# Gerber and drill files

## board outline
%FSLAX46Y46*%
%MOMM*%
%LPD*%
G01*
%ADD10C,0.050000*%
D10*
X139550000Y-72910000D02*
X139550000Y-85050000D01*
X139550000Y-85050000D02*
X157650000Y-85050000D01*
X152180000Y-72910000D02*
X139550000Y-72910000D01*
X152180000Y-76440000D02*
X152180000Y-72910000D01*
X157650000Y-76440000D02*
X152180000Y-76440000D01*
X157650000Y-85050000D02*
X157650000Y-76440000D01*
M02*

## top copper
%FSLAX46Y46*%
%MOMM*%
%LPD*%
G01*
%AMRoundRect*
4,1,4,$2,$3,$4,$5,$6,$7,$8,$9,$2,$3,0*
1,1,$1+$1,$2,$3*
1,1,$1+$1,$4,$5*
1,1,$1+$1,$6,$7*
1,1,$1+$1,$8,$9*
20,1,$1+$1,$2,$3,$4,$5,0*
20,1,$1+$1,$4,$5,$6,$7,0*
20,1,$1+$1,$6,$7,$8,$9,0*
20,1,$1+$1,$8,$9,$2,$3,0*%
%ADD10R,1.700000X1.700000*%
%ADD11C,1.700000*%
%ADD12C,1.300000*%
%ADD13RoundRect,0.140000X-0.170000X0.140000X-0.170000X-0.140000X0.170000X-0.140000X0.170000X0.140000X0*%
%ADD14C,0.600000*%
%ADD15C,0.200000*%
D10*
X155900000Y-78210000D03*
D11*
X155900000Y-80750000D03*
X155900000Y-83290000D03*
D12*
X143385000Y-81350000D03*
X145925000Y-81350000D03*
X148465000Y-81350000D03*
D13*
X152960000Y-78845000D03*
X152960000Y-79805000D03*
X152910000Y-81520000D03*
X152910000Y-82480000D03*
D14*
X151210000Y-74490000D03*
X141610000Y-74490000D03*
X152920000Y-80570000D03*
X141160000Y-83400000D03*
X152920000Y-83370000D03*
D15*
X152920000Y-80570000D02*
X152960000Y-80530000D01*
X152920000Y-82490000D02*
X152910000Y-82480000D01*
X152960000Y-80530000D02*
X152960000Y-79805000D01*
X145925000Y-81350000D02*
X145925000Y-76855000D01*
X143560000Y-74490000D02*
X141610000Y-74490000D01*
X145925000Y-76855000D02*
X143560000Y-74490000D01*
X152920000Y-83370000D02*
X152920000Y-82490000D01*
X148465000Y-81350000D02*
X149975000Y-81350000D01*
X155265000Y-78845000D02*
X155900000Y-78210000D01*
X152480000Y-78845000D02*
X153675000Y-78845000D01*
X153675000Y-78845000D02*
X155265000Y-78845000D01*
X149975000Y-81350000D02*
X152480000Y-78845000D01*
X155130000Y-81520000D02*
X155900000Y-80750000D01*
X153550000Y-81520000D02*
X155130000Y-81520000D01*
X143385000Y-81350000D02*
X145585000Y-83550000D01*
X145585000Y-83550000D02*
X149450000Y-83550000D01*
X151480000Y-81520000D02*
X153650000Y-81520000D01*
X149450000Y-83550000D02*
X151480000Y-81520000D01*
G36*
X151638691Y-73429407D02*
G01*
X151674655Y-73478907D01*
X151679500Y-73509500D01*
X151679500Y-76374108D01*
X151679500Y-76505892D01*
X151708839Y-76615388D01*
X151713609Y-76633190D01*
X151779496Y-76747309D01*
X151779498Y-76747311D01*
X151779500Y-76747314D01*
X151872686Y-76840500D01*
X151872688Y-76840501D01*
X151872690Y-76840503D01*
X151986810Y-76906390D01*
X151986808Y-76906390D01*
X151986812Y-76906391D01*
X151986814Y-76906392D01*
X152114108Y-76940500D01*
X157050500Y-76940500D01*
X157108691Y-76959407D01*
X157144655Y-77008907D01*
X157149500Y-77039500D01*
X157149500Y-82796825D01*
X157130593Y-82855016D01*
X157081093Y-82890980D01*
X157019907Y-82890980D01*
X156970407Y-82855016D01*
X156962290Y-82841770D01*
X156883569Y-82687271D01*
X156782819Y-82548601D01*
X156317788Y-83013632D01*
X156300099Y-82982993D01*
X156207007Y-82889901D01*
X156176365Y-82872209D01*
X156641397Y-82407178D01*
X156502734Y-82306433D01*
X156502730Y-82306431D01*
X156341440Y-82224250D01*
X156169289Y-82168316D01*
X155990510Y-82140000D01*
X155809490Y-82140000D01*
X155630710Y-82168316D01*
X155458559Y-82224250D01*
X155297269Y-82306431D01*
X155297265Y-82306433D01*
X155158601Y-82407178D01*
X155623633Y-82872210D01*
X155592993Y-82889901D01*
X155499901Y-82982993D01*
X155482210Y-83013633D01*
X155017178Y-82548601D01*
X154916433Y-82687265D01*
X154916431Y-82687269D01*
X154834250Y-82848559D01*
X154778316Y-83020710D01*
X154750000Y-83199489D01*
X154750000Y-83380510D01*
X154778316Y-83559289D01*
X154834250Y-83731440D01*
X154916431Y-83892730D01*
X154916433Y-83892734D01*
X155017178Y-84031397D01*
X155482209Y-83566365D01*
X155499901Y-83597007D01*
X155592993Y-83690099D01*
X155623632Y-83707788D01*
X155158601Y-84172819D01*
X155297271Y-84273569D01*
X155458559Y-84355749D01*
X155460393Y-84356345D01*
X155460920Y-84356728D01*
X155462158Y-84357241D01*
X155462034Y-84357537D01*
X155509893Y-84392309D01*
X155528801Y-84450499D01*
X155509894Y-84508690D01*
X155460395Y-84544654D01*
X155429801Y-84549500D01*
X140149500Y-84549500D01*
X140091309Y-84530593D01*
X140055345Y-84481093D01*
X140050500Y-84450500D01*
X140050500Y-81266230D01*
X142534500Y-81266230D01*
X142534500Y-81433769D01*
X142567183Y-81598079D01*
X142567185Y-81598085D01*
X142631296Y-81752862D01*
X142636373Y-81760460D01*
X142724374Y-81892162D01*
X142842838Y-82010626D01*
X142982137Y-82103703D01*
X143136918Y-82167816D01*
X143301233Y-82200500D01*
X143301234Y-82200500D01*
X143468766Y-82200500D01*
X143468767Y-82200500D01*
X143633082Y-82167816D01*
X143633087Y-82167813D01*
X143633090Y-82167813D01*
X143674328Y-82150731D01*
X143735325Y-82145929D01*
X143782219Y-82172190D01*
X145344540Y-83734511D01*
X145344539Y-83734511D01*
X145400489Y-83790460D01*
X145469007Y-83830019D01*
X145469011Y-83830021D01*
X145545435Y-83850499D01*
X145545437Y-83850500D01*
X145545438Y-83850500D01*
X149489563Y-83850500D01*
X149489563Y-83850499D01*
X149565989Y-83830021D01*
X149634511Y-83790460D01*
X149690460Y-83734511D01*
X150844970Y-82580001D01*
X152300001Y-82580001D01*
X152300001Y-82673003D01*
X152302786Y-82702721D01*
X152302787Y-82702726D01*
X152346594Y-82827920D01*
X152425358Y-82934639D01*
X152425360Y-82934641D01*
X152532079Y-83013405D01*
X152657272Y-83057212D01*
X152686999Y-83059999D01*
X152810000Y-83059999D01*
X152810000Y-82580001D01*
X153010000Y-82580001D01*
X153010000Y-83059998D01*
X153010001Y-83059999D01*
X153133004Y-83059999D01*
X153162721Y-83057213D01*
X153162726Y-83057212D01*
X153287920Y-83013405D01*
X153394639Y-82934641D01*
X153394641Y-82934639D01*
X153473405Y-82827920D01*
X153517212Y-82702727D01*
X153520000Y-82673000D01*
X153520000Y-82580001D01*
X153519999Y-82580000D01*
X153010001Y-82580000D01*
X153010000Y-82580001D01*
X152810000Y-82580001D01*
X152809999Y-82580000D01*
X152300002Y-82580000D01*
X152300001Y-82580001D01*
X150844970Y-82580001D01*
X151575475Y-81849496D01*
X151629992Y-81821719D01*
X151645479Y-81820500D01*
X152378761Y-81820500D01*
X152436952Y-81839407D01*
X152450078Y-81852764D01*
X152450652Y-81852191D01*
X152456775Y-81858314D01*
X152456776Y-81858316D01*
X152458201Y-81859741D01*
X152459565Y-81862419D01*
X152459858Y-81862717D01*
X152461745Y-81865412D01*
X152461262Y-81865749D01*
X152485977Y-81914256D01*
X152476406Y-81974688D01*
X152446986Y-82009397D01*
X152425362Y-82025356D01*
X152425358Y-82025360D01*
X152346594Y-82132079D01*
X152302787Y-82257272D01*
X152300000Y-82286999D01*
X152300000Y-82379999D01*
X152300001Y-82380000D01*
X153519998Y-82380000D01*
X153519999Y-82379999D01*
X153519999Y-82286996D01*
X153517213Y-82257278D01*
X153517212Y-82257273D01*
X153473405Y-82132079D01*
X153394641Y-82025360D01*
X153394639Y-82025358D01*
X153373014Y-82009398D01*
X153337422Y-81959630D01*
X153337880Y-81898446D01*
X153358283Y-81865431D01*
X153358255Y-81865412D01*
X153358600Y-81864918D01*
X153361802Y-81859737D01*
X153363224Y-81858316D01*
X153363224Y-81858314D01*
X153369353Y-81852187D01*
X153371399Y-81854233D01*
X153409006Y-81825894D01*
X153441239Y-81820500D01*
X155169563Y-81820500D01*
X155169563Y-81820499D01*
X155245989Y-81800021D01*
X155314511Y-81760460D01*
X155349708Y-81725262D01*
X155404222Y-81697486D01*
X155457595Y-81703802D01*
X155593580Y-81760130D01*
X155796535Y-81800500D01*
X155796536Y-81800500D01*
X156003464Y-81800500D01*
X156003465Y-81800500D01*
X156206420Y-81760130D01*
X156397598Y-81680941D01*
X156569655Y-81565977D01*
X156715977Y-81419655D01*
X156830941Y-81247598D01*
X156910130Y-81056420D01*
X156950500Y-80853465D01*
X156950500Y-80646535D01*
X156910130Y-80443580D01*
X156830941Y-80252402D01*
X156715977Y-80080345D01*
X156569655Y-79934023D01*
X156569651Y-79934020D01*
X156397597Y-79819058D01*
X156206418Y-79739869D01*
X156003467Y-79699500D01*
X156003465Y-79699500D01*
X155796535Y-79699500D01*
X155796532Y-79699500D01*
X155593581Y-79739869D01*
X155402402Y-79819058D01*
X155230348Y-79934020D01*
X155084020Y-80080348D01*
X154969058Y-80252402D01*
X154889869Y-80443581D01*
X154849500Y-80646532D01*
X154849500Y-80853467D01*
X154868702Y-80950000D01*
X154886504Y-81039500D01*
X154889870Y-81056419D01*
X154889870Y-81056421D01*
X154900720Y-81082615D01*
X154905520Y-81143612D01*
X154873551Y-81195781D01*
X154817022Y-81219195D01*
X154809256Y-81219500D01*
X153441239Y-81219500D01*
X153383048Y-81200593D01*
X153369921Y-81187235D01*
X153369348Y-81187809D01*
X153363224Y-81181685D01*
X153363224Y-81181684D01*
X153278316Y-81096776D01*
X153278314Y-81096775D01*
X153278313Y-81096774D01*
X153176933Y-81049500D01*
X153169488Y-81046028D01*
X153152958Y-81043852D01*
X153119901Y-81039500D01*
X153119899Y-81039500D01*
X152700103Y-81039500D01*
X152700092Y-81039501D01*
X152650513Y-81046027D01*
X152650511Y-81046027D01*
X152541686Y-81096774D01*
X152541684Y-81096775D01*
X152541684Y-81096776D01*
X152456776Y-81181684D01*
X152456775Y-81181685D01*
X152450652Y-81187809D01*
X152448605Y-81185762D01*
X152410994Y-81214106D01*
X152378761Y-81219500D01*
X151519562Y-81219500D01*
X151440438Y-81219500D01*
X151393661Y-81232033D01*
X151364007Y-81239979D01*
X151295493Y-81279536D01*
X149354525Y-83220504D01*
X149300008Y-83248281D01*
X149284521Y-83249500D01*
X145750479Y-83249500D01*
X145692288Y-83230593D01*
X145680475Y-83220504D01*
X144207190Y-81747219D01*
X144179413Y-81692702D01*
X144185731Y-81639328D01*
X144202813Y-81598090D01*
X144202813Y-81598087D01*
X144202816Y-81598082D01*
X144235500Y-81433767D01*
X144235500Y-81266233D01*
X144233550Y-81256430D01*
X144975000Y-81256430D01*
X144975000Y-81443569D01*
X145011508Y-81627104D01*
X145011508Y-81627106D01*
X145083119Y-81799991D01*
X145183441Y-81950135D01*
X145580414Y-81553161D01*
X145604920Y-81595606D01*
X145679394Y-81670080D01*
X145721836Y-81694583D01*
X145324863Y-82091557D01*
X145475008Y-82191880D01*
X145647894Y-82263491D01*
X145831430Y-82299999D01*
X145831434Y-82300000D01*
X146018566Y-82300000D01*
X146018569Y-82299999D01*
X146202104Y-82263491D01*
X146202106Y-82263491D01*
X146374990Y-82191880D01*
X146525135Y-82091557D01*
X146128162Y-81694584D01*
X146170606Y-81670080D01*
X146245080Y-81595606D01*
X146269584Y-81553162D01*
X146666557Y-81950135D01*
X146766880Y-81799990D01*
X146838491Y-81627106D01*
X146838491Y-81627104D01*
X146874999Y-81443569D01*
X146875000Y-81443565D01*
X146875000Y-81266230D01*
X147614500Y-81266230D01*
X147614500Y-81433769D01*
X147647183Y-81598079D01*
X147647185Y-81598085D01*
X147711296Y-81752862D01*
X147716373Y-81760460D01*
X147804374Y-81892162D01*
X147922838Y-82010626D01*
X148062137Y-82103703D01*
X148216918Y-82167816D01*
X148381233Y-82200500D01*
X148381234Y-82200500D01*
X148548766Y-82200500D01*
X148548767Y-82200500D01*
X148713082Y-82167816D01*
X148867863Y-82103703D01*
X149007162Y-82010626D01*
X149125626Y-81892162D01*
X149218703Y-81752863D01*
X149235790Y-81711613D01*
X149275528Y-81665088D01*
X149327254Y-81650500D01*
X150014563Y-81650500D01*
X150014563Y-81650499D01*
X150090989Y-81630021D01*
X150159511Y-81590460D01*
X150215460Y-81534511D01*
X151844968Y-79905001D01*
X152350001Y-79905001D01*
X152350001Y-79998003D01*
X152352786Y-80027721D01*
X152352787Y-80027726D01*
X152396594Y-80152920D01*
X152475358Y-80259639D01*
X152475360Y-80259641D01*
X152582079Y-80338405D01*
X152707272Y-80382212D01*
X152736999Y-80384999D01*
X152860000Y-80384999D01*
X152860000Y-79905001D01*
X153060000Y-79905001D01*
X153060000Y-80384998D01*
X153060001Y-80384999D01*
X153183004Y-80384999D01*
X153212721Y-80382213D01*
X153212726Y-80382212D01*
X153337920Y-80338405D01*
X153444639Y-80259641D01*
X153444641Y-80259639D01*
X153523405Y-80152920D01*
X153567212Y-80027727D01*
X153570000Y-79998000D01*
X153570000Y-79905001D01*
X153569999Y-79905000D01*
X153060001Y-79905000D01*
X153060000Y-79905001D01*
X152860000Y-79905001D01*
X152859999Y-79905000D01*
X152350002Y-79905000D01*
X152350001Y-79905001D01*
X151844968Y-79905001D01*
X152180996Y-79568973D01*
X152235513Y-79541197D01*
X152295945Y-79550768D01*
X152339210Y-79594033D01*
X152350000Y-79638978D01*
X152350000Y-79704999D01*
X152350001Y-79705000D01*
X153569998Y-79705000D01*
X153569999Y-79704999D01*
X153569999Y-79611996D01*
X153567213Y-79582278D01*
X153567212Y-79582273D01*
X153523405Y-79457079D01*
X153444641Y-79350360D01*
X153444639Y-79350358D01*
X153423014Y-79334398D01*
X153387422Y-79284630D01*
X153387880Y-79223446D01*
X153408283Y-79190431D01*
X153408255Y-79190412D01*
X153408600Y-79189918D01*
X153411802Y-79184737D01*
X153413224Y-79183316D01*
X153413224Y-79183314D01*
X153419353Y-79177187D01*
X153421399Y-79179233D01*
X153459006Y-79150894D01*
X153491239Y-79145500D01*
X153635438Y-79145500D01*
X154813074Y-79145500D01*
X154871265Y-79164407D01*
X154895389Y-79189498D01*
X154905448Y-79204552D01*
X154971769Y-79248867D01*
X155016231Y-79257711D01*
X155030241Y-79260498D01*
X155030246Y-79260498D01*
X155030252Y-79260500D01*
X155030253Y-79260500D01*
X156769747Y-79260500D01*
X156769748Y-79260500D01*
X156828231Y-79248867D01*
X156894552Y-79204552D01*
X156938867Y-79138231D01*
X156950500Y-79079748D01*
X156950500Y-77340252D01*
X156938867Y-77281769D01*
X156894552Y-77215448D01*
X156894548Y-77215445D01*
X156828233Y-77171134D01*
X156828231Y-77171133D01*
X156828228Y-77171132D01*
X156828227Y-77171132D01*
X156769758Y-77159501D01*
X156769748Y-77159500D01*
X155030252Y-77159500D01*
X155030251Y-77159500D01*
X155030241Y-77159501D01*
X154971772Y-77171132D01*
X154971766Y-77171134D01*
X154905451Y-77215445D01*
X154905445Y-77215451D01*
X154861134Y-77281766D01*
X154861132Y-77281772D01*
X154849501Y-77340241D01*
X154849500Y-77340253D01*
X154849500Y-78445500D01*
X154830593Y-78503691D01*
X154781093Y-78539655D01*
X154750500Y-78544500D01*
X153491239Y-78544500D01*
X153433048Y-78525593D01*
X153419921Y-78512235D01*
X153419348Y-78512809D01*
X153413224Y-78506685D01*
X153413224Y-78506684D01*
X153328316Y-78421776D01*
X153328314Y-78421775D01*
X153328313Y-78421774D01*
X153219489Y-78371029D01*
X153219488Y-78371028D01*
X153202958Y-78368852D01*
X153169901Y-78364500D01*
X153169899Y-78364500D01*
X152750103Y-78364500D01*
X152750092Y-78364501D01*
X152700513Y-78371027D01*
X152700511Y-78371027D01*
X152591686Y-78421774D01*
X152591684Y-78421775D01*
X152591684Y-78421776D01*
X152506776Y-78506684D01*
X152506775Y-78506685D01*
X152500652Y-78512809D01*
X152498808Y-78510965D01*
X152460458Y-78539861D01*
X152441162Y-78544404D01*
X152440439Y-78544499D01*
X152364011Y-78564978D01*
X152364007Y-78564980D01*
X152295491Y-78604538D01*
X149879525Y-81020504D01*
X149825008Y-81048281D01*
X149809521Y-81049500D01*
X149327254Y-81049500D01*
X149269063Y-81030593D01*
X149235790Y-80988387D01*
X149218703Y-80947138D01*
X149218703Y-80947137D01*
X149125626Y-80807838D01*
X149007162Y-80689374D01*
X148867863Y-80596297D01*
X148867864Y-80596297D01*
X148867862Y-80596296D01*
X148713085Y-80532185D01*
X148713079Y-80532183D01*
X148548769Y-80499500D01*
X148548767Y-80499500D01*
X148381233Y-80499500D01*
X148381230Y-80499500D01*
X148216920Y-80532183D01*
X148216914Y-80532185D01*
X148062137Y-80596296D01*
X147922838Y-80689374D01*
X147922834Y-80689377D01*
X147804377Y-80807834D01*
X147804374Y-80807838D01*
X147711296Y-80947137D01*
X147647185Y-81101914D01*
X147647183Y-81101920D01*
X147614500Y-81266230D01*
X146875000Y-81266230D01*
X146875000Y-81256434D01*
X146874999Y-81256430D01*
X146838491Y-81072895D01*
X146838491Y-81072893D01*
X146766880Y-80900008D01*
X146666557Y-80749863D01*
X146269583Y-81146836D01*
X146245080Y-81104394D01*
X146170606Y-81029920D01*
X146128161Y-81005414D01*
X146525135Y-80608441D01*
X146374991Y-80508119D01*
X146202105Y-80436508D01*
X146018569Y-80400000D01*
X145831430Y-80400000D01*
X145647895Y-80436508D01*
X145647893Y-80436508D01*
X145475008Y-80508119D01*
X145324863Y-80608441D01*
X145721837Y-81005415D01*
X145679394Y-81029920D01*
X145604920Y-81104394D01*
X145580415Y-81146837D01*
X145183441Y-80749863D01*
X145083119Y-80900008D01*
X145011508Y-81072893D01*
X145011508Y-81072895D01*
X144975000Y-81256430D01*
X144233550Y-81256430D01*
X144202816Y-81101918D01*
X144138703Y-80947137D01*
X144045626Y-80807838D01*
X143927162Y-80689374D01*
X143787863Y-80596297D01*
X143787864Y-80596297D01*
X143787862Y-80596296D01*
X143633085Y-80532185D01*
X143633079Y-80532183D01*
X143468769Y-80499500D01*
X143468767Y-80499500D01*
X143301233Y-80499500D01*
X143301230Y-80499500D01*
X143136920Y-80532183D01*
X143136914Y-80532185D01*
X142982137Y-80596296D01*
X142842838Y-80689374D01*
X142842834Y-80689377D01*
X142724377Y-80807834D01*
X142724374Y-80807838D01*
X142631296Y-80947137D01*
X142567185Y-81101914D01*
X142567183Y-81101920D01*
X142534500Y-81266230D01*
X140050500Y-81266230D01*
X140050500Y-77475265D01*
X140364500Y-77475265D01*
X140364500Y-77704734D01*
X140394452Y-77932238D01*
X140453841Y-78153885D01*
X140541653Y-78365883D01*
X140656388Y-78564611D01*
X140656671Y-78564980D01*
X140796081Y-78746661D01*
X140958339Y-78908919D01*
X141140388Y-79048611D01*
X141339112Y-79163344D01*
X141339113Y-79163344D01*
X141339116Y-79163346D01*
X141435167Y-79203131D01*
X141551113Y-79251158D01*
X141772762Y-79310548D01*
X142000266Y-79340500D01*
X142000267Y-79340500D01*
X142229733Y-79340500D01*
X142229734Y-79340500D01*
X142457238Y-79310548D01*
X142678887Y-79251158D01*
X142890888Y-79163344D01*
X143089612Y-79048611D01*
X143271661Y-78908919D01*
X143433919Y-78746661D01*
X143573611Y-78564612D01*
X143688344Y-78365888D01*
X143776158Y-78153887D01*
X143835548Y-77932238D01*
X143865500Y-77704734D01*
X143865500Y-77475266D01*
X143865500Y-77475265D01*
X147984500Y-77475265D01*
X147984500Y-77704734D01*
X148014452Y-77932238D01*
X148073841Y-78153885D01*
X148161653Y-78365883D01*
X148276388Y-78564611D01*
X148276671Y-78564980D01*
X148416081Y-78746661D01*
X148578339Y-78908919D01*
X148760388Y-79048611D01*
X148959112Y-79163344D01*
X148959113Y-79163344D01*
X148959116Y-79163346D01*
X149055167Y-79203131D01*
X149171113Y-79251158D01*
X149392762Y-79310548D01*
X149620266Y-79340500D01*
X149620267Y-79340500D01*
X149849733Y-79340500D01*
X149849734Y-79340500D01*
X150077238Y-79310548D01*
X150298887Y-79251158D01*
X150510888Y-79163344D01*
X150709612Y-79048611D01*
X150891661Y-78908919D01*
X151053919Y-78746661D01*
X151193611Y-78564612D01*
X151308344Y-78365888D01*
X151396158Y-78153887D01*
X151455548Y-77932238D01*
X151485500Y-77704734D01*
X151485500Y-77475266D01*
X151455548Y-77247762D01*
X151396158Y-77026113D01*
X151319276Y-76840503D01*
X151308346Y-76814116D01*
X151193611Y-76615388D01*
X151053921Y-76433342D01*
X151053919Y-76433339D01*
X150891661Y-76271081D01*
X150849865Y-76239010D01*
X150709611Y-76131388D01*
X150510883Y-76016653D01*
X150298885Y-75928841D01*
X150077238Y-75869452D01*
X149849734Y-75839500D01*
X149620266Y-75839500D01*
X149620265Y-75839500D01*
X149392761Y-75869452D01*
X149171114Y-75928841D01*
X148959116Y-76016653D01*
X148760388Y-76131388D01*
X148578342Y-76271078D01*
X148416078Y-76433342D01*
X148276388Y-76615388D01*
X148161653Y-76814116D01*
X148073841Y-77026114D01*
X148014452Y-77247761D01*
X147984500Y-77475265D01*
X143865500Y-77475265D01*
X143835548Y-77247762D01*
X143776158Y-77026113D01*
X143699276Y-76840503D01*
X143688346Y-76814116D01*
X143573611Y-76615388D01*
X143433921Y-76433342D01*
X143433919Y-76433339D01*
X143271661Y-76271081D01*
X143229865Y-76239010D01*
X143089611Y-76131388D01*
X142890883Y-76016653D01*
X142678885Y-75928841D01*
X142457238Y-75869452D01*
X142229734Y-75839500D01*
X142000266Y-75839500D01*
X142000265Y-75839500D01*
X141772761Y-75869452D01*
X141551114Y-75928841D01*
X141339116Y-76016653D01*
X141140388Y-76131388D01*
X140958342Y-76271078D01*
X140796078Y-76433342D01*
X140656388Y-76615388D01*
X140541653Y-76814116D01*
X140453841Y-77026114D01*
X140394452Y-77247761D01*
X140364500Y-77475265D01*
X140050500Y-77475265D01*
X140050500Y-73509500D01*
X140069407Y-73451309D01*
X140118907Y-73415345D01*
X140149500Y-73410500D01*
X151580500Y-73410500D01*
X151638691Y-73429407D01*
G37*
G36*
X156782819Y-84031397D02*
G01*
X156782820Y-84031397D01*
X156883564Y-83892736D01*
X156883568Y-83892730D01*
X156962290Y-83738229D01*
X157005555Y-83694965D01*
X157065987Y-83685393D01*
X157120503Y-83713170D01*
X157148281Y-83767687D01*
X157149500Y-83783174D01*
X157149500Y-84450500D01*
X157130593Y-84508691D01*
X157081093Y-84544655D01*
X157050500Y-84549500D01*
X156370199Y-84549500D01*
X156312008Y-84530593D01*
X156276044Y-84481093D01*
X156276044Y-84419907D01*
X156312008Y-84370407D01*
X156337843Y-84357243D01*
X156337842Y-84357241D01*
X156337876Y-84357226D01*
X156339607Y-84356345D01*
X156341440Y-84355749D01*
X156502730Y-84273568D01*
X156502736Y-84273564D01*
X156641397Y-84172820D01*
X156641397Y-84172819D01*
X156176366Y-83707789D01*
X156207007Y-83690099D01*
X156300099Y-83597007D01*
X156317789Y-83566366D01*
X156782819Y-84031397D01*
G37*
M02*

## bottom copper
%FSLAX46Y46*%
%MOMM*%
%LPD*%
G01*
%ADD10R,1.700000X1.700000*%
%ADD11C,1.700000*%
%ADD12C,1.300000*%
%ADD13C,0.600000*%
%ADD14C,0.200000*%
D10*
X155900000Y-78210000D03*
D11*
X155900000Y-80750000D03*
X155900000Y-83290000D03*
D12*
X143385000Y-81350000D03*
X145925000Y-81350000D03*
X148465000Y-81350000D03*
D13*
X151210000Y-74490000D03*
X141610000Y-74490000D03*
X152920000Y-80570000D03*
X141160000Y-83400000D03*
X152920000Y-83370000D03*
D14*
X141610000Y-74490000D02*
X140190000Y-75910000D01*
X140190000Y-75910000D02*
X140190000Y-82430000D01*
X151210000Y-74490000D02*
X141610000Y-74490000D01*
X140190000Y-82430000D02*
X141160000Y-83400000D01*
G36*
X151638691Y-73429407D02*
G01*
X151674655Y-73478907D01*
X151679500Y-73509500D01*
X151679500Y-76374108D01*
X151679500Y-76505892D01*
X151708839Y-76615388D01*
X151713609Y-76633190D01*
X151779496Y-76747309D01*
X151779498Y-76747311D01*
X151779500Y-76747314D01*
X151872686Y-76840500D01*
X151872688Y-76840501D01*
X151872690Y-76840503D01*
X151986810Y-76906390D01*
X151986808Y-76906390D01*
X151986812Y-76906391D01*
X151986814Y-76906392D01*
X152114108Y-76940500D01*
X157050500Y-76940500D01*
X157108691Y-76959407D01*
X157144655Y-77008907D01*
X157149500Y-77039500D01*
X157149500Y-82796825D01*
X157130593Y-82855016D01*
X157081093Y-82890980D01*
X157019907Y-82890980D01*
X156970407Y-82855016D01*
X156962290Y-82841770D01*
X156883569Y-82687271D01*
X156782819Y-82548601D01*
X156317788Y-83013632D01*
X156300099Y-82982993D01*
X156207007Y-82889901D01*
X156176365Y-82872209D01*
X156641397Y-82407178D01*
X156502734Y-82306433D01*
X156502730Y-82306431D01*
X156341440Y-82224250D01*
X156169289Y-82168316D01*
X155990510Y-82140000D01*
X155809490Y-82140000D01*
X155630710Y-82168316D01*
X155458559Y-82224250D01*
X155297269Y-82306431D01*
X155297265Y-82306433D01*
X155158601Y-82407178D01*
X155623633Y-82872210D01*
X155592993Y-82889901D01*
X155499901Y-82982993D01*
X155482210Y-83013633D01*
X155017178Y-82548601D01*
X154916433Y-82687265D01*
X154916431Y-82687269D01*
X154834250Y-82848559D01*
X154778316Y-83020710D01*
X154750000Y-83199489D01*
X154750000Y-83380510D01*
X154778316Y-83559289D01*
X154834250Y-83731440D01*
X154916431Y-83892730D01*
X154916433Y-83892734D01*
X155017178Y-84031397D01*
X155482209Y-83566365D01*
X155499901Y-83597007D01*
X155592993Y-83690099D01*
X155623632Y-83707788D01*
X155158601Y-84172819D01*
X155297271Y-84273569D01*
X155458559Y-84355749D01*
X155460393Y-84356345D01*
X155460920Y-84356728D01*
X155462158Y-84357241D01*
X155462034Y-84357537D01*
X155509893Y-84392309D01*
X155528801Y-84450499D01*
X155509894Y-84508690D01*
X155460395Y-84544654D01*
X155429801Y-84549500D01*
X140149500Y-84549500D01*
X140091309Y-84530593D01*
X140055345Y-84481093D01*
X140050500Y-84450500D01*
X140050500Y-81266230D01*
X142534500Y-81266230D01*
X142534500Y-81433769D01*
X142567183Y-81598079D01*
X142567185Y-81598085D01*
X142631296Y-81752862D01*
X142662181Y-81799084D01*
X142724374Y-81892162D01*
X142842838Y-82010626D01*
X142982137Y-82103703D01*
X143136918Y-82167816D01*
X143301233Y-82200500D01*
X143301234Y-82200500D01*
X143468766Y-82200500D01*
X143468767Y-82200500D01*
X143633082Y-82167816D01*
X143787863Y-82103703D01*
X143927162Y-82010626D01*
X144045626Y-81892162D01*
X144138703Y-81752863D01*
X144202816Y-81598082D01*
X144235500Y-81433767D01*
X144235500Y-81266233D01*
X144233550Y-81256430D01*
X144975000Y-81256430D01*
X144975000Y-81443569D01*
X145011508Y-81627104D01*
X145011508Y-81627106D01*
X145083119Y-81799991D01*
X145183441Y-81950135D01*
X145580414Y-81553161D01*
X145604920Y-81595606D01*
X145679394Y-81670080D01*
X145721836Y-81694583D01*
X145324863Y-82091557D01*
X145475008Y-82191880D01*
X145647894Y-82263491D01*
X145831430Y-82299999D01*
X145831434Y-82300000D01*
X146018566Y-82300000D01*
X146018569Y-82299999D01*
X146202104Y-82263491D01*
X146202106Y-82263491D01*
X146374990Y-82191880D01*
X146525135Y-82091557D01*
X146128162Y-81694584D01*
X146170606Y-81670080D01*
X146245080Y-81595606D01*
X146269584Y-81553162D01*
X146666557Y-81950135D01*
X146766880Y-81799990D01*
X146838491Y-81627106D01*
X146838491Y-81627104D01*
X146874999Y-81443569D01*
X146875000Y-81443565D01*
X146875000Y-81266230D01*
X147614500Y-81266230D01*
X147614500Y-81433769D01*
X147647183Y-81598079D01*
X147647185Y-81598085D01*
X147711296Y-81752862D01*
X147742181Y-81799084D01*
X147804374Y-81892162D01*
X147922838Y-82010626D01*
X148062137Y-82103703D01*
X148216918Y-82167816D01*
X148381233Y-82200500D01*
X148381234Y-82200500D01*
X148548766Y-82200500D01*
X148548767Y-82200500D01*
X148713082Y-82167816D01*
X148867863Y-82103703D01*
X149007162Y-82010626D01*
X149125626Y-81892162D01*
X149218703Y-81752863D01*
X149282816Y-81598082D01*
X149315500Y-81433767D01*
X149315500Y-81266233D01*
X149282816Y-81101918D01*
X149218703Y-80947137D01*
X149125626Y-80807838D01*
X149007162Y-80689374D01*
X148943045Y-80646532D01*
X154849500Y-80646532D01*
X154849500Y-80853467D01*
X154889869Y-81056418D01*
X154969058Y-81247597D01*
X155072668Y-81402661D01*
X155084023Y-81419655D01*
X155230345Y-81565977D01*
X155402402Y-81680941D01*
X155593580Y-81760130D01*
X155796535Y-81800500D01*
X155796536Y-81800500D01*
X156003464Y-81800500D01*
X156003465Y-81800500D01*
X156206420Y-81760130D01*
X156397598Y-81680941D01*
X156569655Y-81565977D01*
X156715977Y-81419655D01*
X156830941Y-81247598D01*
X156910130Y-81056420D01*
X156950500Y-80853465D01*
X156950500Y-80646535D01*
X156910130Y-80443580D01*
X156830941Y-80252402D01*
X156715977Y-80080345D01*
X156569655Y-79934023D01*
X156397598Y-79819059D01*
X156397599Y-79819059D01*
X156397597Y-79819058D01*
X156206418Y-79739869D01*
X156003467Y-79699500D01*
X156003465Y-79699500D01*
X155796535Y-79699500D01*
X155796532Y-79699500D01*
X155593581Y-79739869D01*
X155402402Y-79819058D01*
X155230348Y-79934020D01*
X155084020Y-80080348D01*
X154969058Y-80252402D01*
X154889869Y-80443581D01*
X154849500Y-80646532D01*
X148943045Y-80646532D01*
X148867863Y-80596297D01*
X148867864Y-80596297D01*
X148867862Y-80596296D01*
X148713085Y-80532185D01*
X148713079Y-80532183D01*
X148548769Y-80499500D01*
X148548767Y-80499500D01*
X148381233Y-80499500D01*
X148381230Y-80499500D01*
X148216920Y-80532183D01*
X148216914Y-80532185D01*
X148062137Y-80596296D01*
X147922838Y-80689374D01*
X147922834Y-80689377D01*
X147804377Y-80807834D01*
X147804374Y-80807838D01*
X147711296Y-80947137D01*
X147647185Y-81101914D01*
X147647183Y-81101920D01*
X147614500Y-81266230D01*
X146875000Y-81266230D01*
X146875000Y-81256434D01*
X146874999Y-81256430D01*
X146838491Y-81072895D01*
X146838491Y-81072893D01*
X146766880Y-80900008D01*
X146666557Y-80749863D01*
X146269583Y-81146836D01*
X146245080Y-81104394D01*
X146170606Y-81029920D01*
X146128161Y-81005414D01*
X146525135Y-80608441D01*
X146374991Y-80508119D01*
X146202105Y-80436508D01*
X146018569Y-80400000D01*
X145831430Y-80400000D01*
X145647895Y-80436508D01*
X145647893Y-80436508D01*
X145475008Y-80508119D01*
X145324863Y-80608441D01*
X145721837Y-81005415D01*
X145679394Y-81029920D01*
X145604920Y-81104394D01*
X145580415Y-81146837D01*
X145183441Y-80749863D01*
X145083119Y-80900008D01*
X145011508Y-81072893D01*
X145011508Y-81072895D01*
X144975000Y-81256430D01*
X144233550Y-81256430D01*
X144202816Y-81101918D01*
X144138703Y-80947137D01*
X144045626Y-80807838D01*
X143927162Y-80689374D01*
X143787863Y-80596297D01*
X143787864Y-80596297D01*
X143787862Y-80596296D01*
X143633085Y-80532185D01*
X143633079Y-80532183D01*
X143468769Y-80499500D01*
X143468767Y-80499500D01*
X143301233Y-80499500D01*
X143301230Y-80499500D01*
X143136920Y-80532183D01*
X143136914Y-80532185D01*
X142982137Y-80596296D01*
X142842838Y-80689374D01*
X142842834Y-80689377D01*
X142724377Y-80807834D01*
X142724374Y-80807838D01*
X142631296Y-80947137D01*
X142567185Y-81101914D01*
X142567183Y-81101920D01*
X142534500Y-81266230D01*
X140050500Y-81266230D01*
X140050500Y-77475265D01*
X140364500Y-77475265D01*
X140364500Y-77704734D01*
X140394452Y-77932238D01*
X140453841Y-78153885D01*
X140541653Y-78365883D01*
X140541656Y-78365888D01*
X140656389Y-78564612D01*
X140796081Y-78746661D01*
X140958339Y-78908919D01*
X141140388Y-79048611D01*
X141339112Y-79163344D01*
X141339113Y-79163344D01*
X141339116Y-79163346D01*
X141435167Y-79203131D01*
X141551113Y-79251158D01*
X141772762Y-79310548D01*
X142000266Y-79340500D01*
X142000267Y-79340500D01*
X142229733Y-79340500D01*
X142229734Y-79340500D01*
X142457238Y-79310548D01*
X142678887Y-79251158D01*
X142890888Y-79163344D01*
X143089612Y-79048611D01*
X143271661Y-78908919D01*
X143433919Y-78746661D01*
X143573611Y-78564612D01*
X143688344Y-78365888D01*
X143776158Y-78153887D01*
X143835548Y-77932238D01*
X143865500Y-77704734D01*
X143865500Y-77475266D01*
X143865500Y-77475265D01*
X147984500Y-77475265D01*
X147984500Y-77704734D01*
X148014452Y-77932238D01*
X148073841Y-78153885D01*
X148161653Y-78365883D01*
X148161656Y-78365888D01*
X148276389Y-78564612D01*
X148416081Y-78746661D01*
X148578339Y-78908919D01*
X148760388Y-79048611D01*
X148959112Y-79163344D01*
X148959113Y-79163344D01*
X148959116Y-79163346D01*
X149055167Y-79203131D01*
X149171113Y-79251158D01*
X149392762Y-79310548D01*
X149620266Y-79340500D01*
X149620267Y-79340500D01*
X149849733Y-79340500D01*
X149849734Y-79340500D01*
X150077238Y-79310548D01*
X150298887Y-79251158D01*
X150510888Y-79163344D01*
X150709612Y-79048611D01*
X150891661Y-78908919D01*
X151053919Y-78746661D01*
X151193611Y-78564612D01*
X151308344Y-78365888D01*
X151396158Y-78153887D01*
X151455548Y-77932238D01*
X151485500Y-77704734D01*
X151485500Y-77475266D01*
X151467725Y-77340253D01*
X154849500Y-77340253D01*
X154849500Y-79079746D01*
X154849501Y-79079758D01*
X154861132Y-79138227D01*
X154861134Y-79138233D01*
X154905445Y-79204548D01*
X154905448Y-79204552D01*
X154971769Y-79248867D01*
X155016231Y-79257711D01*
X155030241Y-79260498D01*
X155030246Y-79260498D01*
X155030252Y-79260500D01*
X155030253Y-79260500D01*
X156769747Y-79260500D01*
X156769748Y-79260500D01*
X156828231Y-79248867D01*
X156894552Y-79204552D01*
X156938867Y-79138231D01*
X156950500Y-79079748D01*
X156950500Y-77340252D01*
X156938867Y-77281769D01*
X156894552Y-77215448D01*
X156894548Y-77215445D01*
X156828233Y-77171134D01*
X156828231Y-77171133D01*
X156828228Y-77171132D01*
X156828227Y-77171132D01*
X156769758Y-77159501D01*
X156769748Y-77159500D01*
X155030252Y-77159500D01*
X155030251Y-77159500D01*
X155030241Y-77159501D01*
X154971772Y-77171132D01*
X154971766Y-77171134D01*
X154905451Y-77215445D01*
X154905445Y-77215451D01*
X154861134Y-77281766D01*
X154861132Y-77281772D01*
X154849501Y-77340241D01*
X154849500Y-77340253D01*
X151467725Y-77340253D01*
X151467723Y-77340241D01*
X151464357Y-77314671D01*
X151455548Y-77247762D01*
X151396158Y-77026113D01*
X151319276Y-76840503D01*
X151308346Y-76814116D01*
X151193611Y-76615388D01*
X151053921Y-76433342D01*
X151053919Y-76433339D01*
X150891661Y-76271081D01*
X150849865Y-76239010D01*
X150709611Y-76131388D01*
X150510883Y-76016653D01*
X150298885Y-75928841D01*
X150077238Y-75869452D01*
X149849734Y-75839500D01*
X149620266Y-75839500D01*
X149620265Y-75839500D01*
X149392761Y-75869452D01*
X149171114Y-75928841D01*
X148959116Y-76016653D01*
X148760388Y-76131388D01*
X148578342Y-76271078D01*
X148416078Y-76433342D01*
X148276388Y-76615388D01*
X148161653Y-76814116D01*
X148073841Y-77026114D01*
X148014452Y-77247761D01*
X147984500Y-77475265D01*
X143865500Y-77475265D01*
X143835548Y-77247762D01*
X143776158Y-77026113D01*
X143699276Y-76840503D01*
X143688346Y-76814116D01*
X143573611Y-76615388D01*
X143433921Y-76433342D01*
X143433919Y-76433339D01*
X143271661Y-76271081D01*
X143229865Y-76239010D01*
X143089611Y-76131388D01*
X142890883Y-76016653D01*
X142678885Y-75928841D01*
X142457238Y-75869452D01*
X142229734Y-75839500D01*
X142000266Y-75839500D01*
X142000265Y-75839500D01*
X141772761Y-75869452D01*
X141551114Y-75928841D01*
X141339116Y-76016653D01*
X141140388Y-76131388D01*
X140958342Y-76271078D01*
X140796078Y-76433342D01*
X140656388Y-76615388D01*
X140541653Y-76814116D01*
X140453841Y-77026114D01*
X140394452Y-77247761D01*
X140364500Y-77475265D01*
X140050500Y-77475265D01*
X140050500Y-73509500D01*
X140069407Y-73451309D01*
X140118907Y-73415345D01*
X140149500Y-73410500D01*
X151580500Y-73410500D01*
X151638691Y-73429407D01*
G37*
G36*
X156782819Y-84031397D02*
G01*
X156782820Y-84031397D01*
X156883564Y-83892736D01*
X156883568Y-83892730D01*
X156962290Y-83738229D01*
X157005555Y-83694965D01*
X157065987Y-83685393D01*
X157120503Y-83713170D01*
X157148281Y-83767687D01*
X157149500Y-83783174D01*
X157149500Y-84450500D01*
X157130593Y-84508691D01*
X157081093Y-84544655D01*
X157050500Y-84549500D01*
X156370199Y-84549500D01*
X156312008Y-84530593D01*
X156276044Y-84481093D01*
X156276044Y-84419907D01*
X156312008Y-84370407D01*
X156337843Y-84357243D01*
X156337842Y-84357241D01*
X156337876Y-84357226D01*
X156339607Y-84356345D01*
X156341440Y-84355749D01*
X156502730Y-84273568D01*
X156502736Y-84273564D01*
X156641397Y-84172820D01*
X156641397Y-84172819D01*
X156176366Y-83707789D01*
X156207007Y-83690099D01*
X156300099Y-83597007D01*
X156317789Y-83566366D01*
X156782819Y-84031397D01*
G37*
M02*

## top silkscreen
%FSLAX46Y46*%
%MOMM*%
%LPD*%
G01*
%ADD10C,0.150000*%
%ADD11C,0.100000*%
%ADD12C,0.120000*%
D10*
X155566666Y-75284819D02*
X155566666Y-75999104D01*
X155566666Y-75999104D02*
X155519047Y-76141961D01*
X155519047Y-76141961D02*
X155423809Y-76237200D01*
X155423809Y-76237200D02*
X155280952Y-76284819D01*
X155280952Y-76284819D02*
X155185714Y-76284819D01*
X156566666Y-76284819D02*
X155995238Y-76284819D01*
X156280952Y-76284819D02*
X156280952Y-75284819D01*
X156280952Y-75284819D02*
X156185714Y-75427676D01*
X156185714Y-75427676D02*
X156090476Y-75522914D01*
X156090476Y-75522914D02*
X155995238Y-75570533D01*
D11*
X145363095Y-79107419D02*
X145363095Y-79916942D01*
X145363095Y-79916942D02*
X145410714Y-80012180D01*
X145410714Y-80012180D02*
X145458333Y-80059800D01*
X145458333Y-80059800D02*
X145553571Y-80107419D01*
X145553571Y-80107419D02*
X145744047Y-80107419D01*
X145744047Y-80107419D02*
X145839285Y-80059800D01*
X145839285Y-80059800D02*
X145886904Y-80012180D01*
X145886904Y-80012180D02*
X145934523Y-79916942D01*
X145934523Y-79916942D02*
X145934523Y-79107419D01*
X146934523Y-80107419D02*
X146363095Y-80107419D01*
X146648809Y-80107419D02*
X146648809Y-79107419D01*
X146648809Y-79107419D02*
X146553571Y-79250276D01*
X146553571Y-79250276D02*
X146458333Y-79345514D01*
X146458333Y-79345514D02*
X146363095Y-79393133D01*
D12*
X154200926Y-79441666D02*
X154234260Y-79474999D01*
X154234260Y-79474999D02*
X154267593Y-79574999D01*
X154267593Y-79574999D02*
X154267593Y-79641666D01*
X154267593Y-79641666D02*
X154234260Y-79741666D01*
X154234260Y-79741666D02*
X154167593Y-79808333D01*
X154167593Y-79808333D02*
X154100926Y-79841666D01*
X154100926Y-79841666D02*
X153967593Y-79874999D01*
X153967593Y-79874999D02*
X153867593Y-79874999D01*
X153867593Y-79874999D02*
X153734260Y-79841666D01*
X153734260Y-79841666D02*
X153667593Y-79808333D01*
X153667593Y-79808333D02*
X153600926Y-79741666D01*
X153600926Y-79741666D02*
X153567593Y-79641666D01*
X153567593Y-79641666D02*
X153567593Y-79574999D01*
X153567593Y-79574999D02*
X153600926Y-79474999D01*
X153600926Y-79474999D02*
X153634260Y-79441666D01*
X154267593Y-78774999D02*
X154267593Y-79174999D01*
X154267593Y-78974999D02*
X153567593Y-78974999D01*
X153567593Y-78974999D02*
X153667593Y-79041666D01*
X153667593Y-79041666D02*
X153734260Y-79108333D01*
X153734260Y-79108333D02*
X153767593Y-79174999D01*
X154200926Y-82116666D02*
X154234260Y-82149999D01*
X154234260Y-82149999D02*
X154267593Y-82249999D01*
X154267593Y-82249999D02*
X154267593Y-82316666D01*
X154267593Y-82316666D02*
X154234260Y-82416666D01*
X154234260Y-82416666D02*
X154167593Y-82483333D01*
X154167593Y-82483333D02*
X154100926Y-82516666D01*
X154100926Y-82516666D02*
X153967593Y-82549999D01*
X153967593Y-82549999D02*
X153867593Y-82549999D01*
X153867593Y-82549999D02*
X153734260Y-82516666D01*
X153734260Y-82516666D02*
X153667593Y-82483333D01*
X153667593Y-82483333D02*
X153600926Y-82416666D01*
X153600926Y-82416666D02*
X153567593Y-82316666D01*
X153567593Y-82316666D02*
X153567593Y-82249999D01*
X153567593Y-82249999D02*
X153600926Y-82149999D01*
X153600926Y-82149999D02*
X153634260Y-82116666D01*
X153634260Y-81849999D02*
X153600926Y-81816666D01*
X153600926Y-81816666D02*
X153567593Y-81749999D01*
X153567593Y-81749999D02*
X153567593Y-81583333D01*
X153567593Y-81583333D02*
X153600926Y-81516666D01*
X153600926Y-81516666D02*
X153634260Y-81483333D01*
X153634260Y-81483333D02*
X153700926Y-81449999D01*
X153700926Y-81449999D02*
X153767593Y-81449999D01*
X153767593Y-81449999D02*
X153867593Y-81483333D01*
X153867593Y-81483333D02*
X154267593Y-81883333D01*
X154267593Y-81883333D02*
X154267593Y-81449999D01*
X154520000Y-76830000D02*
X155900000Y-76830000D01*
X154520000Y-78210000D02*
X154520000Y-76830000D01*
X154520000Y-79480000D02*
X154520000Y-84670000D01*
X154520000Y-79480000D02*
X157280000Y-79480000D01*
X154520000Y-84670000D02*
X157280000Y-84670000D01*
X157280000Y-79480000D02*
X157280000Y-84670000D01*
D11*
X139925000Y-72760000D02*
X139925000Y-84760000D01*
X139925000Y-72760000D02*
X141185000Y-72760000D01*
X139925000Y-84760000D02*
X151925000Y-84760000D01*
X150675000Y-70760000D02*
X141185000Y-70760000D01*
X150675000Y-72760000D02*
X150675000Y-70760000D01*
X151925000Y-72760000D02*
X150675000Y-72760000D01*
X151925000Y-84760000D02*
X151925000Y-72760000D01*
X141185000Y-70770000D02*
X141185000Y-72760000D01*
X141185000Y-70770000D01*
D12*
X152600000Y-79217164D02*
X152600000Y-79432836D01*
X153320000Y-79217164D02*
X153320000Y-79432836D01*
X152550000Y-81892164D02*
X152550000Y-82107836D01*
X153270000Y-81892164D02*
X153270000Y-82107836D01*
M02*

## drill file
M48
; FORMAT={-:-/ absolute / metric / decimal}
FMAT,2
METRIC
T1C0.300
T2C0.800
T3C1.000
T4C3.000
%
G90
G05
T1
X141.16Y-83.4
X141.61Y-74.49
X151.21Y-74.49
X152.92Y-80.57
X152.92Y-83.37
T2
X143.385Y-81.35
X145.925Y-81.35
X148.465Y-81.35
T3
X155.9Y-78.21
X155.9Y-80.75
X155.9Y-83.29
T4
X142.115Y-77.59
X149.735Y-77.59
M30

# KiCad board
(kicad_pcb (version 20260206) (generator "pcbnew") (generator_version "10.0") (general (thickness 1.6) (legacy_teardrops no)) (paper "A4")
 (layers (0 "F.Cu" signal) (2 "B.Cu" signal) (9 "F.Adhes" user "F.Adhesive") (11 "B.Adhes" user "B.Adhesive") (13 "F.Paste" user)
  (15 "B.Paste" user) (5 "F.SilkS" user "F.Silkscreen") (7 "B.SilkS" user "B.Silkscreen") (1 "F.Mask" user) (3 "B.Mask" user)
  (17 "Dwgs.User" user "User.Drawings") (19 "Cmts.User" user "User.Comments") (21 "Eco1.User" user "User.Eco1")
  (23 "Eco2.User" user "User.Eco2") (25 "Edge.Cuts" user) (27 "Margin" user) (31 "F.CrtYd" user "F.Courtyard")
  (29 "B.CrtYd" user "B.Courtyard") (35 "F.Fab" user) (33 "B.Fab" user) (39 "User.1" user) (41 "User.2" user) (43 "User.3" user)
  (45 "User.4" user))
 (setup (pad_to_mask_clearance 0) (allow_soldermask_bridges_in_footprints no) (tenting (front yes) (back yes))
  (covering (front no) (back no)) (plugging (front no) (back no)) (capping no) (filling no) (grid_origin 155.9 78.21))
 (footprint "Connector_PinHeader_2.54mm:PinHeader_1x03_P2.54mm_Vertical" (layer "F.Cu") (at 155.9 78.21)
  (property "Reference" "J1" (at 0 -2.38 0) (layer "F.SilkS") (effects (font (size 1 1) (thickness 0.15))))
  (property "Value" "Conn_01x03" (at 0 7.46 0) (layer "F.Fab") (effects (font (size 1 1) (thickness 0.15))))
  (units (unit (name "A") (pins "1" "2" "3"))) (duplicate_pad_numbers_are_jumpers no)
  (fp_line (start -1.38 -1.38) (end 0 -1.38) (stroke (width 0.12) (type solid)) (layer "F.SilkS"))
  (fp_line (start -1.38 0) (end -1.38 -1.38) (stroke (width 0.12) (type solid)) (layer "F.SilkS"))
  (fp_line (start -1.38 1.27) (end -1.38 6.46) (stroke (width 0.12) (type solid)) (layer "F.SilkS"))
  (fp_line (start -1.38 1.27) (end 1.38 1.27) (stroke (width 0.12) (type solid)) (layer "F.SilkS"))
  (fp_line (start -1.38 6.46) (end 1.38 6.46) (stroke (width 0.12) (type solid)) (layer "F.SilkS"))
  (fp_line (start 1.38 1.27) (end 1.38 6.46) (stroke (width 0.12) (type solid)) (layer "F.SilkS"))
  (pad "1" thru_hole rect (at 0 0) (size 1.7 1.7) (drill 1) (layers "*.Cu" "*.Mask") (remove_unused_layers no) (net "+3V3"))
  (pad "2" thru_hole circle (at 0 2.54) (size 1.7 1.7) (drill 1) (layers "*.Cu" "*.Mask") (remove_unused_layers no) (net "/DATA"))
  (pad "3" thru_hole circle (at 0 5.08) (size 1.7 1.7) (drill 1) (layers "*.Cu" "*.Mask") (remove_unused_layers no) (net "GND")))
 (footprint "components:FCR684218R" (layer "F.Cu") (at 145.925 81.35)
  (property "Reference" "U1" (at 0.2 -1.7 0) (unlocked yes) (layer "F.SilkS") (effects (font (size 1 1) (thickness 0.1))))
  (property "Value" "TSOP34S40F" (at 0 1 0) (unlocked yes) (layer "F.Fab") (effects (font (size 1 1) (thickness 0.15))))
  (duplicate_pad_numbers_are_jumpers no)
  (fp_line (start -6 -8.59) (end -6 3.41) (stroke (width 0.1) (type default)) (layer "F.SilkS"))
  (fp_line (start -6 -8.59) (end -4.74 -8.59) (stroke (width 0.1) (type default)) (layer "F.SilkS"))
  (fp_line (start -6 3.41) (end 6 3.41) (stroke (width 0.1) (type default)) (layer "F.SilkS"))
  (fp_line (start 4.75 -10.59) (end -4.74 -10.59) (stroke (width 0.1) (type default)) (layer "F.SilkS"))
  (fp_line (start 4.75 -8.59) (end 4.75 -10.59) (stroke (width 0.1) (type default)) (layer "F.SilkS"))
  (fp_line (start 6 -8.59) (end 4.75 -8.59) (stroke (width 0.1) (type default)) (layer "F.SilkS"))
  (fp_line (start 6 3.41) (end 6 -8.59) (stroke (width 0.1) (type default)) (layer "F.SilkS"))
  (fp_rect (start -4.74 -10.58) (end -4.74 -8.59) (stroke (width 0.1) (type default)) (fill no) (layer "F.SilkS"))
  (pad "" np_thru_hole circle (at -3.81 -3.76) (size 3 3) (drill 3) (layers "*.Cu" "*.Mask"))
  (pad "" np_thru_hole circle (at 3.81 -3.76) (size 3 3) (drill 3) (layers "*.Cu" "*.Mask"))
  (pad "1" thru_hole circle (at -2.54 0) (size 1.3 1.3) (drill 0.8) (layers "*.Cu" "*.Mask") (remove_unused_layers no) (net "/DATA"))
  (pad "2" thru_hole circle (at 0 0) (size 1.3 1.3) (drill 0.8) (layers "*.Cu" "*.Mask") (remove_unused_layers no) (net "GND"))
  (pad "3" thru_hole circle (at 2.54 0) (size 1.3 1.3) (drill 0.8) (layers "*.Cu" "*.Mask") (remove_unused_layers no) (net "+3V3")))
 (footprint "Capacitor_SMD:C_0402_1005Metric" (layer "F.Cu") (at 152.96 79.325 -90)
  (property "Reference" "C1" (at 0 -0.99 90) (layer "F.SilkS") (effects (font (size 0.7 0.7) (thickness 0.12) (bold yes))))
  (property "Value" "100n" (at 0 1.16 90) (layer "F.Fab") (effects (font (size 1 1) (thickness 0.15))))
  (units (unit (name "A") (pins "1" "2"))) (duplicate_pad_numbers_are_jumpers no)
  (fp_line (start -0.107836 0.36) (end 0.107836 0.36) (stroke (width 0.12) (type solid)) (layer "F.SilkS"))
  (fp_line (start -0.107836 -0.36) (end 0.107836 -0.36) (stroke (width 0.12) (type solid)) (layer "F.SilkS"))
  (pad "1" smd roundrect (at -0.48 0 270) (size 0.56 0.62) (layers "F.Cu" "F.Mask" "F.Paste") (roundrect_rratio 0.25) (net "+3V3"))
  (pad "2" smd roundrect (at 0.48 0 270) (size 0.56 0.62) (layers "F.Cu" "F.Mask" "F.Paste") (roundrect_rratio 0.25) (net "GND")))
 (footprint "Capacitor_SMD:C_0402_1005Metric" (layer "F.Cu") (at 152.91 82 -90)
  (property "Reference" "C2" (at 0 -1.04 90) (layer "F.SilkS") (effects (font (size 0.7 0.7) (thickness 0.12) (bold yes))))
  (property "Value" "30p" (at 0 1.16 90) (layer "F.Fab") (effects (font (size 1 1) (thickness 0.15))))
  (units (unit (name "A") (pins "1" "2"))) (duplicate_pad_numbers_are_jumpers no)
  (fp_line (start -0.107836 0.36) (end 0.107836 0.36) (stroke (width 0.12) (type solid)) (layer "F.SilkS"))
  (fp_line (start -0.107836 -0.36) (end 0.107836 -0.36) (stroke (width 0.12) (type solid)) (layer "F.SilkS"))
  (pad "1" smd roundrect (at -0.48 0 270) (size 0.56 0.62) (layers "F.Cu" "F.Mask" "F.Paste") (roundrect_rratio 0.25) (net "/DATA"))
  (pad "2" smd roundrect (at 0.48 0 270) (size 0.56 0.62) (layers "F.Cu" "F.Mask" "F.Paste") (roundrect_rratio 0.25) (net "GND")))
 (gr_line (start 139.55 72.91) (end 139.55 85.05) (stroke (width 0.05) (type default)) (layer "Edge.Cuts"))
 (gr_line (start 139.55 85.05) (end 157.65 85.05) (stroke (width 0.05) (type default)) (layer "Edge.Cuts"))
 (gr_line (start 152.18 72.91) (end 139.55 72.91) (stroke (width 0.05) (type default)) (layer "Edge.Cuts"))
 (gr_line (start 152.18 76.44) (end 152.18 72.91) (stroke (width 0.05) (type default)) (layer "Edge.Cuts"))
 (gr_line (start 157.65 76.44) (end 152.18 76.44) (stroke (width 0.05) (type default)) (layer "Edge.Cuts"))
 (gr_line (start 157.65 85.05) (end 157.65 76.44) (stroke (width 0.05) (type default)) (layer "Edge.Cuts"))
 (segment (start 152.92 80.57) (end 152.96 80.53) (width 0.2) (layer "F.Cu") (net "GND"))
 (segment (start 152.92 82.49) (end 152.91 82.48) (width 0.2) (layer "F.Cu") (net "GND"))
 (segment (start 152.96 80.53) (end 152.96 79.805) (width 0.2) (layer "F.Cu") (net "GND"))
 (segment (start 145.925 81.35) (end 145.925 76.855) (width 0.2) (layer "F.Cu") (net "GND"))
 (segment (start 143.56 74.49) (end 141.61 74.49) (width 0.2) (layer "F.Cu") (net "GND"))
 (segment (start 145.925 76.855) (end 143.56 74.49) (width 0.2) (layer "F.Cu") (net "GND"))
 (segment (start 152.92 83.37) (end 152.92 82.49) (width 0.2) (layer "F.Cu") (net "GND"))
 (via (at 151.21 74.49) (size 0.6) (drill 0.3) (layers "F.Cu" "B.Cu") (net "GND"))
 (via (at 141.61 74.49) (size 0.6) (drill 0.3) (layers "F.Cu" "B.Cu") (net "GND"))
 (via (at 152.92 80.57) (size 0.6) (drill 0.3) (layers "F.Cu" "B.Cu") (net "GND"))
 (via (at 141.16 83.4) (size 0.6) (drill 0.3) (layers "F.Cu" "B.Cu") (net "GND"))
 (via (at 152.92 83.37) (size 0.6) (drill 0.3) (layers "F.Cu" "B.Cu") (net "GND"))
 (segment (start 141.61 74.49) (end 140.19 75.91) (width 0.2) (layer "B.Cu") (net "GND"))
 (segment (start 140.19 75.91) (end 140.19 82.43) (width 0.2) (layer "B.Cu") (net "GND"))
 (segment (start 151.21 74.49) (end 141.61 74.49) (width 0.2) (layer "B.Cu") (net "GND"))
 (segment (start 140.19 82.43) (end 141.16 83.4) (width 0.2) (layer "B.Cu") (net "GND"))
 (segment (start 148.465 81.35) (end 149.975 81.35) (width 0.2) (layer "F.Cu") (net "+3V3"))
 (segment (start 155.265 78.845) (end 155.9 78.21) (width 0.2) (layer "F.Cu") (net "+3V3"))
 (segment (start 152.48 78.845) (end 153.675 78.845) (width 0.2) (layer "F.Cu") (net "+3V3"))
 (segment (start 153.675 78.845) (end 155.265 78.845) (width 0.2) (layer "F.Cu") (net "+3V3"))
 (segment (start 149.975 81.35) (end 152.48 78.845) (width 0.2) (layer "F.Cu") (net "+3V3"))
 (segment (start 155.13 81.52) (end 155.9 80.75) (width 0.2) (layer "F.Cu") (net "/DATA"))
 (segment (start 153.55 81.52) (end 155.13 81.52) (width 0.2) (layer "F.Cu") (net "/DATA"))
 (segment (start 143.385 81.35) (end 145.585 83.55) (width 0.2) (layer "F.Cu") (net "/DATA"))
 (segment (start 145.585 83.55) (end 149.45 83.55) (width 0.2) (layer "F.Cu") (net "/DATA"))
 (segment (start 151.48 81.52) (end 153.65 81.52) (width 0.2) (layer "F.Cu") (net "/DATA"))
 (segment (start 149.45 83.55) (end 151.48 81.52) (width 0.2) (layer "F.Cu") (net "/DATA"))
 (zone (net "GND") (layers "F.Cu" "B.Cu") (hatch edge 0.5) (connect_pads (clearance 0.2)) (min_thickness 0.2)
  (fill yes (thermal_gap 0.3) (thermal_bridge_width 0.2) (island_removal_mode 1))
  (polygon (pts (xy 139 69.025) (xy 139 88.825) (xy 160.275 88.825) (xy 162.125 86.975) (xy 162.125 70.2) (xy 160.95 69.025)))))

